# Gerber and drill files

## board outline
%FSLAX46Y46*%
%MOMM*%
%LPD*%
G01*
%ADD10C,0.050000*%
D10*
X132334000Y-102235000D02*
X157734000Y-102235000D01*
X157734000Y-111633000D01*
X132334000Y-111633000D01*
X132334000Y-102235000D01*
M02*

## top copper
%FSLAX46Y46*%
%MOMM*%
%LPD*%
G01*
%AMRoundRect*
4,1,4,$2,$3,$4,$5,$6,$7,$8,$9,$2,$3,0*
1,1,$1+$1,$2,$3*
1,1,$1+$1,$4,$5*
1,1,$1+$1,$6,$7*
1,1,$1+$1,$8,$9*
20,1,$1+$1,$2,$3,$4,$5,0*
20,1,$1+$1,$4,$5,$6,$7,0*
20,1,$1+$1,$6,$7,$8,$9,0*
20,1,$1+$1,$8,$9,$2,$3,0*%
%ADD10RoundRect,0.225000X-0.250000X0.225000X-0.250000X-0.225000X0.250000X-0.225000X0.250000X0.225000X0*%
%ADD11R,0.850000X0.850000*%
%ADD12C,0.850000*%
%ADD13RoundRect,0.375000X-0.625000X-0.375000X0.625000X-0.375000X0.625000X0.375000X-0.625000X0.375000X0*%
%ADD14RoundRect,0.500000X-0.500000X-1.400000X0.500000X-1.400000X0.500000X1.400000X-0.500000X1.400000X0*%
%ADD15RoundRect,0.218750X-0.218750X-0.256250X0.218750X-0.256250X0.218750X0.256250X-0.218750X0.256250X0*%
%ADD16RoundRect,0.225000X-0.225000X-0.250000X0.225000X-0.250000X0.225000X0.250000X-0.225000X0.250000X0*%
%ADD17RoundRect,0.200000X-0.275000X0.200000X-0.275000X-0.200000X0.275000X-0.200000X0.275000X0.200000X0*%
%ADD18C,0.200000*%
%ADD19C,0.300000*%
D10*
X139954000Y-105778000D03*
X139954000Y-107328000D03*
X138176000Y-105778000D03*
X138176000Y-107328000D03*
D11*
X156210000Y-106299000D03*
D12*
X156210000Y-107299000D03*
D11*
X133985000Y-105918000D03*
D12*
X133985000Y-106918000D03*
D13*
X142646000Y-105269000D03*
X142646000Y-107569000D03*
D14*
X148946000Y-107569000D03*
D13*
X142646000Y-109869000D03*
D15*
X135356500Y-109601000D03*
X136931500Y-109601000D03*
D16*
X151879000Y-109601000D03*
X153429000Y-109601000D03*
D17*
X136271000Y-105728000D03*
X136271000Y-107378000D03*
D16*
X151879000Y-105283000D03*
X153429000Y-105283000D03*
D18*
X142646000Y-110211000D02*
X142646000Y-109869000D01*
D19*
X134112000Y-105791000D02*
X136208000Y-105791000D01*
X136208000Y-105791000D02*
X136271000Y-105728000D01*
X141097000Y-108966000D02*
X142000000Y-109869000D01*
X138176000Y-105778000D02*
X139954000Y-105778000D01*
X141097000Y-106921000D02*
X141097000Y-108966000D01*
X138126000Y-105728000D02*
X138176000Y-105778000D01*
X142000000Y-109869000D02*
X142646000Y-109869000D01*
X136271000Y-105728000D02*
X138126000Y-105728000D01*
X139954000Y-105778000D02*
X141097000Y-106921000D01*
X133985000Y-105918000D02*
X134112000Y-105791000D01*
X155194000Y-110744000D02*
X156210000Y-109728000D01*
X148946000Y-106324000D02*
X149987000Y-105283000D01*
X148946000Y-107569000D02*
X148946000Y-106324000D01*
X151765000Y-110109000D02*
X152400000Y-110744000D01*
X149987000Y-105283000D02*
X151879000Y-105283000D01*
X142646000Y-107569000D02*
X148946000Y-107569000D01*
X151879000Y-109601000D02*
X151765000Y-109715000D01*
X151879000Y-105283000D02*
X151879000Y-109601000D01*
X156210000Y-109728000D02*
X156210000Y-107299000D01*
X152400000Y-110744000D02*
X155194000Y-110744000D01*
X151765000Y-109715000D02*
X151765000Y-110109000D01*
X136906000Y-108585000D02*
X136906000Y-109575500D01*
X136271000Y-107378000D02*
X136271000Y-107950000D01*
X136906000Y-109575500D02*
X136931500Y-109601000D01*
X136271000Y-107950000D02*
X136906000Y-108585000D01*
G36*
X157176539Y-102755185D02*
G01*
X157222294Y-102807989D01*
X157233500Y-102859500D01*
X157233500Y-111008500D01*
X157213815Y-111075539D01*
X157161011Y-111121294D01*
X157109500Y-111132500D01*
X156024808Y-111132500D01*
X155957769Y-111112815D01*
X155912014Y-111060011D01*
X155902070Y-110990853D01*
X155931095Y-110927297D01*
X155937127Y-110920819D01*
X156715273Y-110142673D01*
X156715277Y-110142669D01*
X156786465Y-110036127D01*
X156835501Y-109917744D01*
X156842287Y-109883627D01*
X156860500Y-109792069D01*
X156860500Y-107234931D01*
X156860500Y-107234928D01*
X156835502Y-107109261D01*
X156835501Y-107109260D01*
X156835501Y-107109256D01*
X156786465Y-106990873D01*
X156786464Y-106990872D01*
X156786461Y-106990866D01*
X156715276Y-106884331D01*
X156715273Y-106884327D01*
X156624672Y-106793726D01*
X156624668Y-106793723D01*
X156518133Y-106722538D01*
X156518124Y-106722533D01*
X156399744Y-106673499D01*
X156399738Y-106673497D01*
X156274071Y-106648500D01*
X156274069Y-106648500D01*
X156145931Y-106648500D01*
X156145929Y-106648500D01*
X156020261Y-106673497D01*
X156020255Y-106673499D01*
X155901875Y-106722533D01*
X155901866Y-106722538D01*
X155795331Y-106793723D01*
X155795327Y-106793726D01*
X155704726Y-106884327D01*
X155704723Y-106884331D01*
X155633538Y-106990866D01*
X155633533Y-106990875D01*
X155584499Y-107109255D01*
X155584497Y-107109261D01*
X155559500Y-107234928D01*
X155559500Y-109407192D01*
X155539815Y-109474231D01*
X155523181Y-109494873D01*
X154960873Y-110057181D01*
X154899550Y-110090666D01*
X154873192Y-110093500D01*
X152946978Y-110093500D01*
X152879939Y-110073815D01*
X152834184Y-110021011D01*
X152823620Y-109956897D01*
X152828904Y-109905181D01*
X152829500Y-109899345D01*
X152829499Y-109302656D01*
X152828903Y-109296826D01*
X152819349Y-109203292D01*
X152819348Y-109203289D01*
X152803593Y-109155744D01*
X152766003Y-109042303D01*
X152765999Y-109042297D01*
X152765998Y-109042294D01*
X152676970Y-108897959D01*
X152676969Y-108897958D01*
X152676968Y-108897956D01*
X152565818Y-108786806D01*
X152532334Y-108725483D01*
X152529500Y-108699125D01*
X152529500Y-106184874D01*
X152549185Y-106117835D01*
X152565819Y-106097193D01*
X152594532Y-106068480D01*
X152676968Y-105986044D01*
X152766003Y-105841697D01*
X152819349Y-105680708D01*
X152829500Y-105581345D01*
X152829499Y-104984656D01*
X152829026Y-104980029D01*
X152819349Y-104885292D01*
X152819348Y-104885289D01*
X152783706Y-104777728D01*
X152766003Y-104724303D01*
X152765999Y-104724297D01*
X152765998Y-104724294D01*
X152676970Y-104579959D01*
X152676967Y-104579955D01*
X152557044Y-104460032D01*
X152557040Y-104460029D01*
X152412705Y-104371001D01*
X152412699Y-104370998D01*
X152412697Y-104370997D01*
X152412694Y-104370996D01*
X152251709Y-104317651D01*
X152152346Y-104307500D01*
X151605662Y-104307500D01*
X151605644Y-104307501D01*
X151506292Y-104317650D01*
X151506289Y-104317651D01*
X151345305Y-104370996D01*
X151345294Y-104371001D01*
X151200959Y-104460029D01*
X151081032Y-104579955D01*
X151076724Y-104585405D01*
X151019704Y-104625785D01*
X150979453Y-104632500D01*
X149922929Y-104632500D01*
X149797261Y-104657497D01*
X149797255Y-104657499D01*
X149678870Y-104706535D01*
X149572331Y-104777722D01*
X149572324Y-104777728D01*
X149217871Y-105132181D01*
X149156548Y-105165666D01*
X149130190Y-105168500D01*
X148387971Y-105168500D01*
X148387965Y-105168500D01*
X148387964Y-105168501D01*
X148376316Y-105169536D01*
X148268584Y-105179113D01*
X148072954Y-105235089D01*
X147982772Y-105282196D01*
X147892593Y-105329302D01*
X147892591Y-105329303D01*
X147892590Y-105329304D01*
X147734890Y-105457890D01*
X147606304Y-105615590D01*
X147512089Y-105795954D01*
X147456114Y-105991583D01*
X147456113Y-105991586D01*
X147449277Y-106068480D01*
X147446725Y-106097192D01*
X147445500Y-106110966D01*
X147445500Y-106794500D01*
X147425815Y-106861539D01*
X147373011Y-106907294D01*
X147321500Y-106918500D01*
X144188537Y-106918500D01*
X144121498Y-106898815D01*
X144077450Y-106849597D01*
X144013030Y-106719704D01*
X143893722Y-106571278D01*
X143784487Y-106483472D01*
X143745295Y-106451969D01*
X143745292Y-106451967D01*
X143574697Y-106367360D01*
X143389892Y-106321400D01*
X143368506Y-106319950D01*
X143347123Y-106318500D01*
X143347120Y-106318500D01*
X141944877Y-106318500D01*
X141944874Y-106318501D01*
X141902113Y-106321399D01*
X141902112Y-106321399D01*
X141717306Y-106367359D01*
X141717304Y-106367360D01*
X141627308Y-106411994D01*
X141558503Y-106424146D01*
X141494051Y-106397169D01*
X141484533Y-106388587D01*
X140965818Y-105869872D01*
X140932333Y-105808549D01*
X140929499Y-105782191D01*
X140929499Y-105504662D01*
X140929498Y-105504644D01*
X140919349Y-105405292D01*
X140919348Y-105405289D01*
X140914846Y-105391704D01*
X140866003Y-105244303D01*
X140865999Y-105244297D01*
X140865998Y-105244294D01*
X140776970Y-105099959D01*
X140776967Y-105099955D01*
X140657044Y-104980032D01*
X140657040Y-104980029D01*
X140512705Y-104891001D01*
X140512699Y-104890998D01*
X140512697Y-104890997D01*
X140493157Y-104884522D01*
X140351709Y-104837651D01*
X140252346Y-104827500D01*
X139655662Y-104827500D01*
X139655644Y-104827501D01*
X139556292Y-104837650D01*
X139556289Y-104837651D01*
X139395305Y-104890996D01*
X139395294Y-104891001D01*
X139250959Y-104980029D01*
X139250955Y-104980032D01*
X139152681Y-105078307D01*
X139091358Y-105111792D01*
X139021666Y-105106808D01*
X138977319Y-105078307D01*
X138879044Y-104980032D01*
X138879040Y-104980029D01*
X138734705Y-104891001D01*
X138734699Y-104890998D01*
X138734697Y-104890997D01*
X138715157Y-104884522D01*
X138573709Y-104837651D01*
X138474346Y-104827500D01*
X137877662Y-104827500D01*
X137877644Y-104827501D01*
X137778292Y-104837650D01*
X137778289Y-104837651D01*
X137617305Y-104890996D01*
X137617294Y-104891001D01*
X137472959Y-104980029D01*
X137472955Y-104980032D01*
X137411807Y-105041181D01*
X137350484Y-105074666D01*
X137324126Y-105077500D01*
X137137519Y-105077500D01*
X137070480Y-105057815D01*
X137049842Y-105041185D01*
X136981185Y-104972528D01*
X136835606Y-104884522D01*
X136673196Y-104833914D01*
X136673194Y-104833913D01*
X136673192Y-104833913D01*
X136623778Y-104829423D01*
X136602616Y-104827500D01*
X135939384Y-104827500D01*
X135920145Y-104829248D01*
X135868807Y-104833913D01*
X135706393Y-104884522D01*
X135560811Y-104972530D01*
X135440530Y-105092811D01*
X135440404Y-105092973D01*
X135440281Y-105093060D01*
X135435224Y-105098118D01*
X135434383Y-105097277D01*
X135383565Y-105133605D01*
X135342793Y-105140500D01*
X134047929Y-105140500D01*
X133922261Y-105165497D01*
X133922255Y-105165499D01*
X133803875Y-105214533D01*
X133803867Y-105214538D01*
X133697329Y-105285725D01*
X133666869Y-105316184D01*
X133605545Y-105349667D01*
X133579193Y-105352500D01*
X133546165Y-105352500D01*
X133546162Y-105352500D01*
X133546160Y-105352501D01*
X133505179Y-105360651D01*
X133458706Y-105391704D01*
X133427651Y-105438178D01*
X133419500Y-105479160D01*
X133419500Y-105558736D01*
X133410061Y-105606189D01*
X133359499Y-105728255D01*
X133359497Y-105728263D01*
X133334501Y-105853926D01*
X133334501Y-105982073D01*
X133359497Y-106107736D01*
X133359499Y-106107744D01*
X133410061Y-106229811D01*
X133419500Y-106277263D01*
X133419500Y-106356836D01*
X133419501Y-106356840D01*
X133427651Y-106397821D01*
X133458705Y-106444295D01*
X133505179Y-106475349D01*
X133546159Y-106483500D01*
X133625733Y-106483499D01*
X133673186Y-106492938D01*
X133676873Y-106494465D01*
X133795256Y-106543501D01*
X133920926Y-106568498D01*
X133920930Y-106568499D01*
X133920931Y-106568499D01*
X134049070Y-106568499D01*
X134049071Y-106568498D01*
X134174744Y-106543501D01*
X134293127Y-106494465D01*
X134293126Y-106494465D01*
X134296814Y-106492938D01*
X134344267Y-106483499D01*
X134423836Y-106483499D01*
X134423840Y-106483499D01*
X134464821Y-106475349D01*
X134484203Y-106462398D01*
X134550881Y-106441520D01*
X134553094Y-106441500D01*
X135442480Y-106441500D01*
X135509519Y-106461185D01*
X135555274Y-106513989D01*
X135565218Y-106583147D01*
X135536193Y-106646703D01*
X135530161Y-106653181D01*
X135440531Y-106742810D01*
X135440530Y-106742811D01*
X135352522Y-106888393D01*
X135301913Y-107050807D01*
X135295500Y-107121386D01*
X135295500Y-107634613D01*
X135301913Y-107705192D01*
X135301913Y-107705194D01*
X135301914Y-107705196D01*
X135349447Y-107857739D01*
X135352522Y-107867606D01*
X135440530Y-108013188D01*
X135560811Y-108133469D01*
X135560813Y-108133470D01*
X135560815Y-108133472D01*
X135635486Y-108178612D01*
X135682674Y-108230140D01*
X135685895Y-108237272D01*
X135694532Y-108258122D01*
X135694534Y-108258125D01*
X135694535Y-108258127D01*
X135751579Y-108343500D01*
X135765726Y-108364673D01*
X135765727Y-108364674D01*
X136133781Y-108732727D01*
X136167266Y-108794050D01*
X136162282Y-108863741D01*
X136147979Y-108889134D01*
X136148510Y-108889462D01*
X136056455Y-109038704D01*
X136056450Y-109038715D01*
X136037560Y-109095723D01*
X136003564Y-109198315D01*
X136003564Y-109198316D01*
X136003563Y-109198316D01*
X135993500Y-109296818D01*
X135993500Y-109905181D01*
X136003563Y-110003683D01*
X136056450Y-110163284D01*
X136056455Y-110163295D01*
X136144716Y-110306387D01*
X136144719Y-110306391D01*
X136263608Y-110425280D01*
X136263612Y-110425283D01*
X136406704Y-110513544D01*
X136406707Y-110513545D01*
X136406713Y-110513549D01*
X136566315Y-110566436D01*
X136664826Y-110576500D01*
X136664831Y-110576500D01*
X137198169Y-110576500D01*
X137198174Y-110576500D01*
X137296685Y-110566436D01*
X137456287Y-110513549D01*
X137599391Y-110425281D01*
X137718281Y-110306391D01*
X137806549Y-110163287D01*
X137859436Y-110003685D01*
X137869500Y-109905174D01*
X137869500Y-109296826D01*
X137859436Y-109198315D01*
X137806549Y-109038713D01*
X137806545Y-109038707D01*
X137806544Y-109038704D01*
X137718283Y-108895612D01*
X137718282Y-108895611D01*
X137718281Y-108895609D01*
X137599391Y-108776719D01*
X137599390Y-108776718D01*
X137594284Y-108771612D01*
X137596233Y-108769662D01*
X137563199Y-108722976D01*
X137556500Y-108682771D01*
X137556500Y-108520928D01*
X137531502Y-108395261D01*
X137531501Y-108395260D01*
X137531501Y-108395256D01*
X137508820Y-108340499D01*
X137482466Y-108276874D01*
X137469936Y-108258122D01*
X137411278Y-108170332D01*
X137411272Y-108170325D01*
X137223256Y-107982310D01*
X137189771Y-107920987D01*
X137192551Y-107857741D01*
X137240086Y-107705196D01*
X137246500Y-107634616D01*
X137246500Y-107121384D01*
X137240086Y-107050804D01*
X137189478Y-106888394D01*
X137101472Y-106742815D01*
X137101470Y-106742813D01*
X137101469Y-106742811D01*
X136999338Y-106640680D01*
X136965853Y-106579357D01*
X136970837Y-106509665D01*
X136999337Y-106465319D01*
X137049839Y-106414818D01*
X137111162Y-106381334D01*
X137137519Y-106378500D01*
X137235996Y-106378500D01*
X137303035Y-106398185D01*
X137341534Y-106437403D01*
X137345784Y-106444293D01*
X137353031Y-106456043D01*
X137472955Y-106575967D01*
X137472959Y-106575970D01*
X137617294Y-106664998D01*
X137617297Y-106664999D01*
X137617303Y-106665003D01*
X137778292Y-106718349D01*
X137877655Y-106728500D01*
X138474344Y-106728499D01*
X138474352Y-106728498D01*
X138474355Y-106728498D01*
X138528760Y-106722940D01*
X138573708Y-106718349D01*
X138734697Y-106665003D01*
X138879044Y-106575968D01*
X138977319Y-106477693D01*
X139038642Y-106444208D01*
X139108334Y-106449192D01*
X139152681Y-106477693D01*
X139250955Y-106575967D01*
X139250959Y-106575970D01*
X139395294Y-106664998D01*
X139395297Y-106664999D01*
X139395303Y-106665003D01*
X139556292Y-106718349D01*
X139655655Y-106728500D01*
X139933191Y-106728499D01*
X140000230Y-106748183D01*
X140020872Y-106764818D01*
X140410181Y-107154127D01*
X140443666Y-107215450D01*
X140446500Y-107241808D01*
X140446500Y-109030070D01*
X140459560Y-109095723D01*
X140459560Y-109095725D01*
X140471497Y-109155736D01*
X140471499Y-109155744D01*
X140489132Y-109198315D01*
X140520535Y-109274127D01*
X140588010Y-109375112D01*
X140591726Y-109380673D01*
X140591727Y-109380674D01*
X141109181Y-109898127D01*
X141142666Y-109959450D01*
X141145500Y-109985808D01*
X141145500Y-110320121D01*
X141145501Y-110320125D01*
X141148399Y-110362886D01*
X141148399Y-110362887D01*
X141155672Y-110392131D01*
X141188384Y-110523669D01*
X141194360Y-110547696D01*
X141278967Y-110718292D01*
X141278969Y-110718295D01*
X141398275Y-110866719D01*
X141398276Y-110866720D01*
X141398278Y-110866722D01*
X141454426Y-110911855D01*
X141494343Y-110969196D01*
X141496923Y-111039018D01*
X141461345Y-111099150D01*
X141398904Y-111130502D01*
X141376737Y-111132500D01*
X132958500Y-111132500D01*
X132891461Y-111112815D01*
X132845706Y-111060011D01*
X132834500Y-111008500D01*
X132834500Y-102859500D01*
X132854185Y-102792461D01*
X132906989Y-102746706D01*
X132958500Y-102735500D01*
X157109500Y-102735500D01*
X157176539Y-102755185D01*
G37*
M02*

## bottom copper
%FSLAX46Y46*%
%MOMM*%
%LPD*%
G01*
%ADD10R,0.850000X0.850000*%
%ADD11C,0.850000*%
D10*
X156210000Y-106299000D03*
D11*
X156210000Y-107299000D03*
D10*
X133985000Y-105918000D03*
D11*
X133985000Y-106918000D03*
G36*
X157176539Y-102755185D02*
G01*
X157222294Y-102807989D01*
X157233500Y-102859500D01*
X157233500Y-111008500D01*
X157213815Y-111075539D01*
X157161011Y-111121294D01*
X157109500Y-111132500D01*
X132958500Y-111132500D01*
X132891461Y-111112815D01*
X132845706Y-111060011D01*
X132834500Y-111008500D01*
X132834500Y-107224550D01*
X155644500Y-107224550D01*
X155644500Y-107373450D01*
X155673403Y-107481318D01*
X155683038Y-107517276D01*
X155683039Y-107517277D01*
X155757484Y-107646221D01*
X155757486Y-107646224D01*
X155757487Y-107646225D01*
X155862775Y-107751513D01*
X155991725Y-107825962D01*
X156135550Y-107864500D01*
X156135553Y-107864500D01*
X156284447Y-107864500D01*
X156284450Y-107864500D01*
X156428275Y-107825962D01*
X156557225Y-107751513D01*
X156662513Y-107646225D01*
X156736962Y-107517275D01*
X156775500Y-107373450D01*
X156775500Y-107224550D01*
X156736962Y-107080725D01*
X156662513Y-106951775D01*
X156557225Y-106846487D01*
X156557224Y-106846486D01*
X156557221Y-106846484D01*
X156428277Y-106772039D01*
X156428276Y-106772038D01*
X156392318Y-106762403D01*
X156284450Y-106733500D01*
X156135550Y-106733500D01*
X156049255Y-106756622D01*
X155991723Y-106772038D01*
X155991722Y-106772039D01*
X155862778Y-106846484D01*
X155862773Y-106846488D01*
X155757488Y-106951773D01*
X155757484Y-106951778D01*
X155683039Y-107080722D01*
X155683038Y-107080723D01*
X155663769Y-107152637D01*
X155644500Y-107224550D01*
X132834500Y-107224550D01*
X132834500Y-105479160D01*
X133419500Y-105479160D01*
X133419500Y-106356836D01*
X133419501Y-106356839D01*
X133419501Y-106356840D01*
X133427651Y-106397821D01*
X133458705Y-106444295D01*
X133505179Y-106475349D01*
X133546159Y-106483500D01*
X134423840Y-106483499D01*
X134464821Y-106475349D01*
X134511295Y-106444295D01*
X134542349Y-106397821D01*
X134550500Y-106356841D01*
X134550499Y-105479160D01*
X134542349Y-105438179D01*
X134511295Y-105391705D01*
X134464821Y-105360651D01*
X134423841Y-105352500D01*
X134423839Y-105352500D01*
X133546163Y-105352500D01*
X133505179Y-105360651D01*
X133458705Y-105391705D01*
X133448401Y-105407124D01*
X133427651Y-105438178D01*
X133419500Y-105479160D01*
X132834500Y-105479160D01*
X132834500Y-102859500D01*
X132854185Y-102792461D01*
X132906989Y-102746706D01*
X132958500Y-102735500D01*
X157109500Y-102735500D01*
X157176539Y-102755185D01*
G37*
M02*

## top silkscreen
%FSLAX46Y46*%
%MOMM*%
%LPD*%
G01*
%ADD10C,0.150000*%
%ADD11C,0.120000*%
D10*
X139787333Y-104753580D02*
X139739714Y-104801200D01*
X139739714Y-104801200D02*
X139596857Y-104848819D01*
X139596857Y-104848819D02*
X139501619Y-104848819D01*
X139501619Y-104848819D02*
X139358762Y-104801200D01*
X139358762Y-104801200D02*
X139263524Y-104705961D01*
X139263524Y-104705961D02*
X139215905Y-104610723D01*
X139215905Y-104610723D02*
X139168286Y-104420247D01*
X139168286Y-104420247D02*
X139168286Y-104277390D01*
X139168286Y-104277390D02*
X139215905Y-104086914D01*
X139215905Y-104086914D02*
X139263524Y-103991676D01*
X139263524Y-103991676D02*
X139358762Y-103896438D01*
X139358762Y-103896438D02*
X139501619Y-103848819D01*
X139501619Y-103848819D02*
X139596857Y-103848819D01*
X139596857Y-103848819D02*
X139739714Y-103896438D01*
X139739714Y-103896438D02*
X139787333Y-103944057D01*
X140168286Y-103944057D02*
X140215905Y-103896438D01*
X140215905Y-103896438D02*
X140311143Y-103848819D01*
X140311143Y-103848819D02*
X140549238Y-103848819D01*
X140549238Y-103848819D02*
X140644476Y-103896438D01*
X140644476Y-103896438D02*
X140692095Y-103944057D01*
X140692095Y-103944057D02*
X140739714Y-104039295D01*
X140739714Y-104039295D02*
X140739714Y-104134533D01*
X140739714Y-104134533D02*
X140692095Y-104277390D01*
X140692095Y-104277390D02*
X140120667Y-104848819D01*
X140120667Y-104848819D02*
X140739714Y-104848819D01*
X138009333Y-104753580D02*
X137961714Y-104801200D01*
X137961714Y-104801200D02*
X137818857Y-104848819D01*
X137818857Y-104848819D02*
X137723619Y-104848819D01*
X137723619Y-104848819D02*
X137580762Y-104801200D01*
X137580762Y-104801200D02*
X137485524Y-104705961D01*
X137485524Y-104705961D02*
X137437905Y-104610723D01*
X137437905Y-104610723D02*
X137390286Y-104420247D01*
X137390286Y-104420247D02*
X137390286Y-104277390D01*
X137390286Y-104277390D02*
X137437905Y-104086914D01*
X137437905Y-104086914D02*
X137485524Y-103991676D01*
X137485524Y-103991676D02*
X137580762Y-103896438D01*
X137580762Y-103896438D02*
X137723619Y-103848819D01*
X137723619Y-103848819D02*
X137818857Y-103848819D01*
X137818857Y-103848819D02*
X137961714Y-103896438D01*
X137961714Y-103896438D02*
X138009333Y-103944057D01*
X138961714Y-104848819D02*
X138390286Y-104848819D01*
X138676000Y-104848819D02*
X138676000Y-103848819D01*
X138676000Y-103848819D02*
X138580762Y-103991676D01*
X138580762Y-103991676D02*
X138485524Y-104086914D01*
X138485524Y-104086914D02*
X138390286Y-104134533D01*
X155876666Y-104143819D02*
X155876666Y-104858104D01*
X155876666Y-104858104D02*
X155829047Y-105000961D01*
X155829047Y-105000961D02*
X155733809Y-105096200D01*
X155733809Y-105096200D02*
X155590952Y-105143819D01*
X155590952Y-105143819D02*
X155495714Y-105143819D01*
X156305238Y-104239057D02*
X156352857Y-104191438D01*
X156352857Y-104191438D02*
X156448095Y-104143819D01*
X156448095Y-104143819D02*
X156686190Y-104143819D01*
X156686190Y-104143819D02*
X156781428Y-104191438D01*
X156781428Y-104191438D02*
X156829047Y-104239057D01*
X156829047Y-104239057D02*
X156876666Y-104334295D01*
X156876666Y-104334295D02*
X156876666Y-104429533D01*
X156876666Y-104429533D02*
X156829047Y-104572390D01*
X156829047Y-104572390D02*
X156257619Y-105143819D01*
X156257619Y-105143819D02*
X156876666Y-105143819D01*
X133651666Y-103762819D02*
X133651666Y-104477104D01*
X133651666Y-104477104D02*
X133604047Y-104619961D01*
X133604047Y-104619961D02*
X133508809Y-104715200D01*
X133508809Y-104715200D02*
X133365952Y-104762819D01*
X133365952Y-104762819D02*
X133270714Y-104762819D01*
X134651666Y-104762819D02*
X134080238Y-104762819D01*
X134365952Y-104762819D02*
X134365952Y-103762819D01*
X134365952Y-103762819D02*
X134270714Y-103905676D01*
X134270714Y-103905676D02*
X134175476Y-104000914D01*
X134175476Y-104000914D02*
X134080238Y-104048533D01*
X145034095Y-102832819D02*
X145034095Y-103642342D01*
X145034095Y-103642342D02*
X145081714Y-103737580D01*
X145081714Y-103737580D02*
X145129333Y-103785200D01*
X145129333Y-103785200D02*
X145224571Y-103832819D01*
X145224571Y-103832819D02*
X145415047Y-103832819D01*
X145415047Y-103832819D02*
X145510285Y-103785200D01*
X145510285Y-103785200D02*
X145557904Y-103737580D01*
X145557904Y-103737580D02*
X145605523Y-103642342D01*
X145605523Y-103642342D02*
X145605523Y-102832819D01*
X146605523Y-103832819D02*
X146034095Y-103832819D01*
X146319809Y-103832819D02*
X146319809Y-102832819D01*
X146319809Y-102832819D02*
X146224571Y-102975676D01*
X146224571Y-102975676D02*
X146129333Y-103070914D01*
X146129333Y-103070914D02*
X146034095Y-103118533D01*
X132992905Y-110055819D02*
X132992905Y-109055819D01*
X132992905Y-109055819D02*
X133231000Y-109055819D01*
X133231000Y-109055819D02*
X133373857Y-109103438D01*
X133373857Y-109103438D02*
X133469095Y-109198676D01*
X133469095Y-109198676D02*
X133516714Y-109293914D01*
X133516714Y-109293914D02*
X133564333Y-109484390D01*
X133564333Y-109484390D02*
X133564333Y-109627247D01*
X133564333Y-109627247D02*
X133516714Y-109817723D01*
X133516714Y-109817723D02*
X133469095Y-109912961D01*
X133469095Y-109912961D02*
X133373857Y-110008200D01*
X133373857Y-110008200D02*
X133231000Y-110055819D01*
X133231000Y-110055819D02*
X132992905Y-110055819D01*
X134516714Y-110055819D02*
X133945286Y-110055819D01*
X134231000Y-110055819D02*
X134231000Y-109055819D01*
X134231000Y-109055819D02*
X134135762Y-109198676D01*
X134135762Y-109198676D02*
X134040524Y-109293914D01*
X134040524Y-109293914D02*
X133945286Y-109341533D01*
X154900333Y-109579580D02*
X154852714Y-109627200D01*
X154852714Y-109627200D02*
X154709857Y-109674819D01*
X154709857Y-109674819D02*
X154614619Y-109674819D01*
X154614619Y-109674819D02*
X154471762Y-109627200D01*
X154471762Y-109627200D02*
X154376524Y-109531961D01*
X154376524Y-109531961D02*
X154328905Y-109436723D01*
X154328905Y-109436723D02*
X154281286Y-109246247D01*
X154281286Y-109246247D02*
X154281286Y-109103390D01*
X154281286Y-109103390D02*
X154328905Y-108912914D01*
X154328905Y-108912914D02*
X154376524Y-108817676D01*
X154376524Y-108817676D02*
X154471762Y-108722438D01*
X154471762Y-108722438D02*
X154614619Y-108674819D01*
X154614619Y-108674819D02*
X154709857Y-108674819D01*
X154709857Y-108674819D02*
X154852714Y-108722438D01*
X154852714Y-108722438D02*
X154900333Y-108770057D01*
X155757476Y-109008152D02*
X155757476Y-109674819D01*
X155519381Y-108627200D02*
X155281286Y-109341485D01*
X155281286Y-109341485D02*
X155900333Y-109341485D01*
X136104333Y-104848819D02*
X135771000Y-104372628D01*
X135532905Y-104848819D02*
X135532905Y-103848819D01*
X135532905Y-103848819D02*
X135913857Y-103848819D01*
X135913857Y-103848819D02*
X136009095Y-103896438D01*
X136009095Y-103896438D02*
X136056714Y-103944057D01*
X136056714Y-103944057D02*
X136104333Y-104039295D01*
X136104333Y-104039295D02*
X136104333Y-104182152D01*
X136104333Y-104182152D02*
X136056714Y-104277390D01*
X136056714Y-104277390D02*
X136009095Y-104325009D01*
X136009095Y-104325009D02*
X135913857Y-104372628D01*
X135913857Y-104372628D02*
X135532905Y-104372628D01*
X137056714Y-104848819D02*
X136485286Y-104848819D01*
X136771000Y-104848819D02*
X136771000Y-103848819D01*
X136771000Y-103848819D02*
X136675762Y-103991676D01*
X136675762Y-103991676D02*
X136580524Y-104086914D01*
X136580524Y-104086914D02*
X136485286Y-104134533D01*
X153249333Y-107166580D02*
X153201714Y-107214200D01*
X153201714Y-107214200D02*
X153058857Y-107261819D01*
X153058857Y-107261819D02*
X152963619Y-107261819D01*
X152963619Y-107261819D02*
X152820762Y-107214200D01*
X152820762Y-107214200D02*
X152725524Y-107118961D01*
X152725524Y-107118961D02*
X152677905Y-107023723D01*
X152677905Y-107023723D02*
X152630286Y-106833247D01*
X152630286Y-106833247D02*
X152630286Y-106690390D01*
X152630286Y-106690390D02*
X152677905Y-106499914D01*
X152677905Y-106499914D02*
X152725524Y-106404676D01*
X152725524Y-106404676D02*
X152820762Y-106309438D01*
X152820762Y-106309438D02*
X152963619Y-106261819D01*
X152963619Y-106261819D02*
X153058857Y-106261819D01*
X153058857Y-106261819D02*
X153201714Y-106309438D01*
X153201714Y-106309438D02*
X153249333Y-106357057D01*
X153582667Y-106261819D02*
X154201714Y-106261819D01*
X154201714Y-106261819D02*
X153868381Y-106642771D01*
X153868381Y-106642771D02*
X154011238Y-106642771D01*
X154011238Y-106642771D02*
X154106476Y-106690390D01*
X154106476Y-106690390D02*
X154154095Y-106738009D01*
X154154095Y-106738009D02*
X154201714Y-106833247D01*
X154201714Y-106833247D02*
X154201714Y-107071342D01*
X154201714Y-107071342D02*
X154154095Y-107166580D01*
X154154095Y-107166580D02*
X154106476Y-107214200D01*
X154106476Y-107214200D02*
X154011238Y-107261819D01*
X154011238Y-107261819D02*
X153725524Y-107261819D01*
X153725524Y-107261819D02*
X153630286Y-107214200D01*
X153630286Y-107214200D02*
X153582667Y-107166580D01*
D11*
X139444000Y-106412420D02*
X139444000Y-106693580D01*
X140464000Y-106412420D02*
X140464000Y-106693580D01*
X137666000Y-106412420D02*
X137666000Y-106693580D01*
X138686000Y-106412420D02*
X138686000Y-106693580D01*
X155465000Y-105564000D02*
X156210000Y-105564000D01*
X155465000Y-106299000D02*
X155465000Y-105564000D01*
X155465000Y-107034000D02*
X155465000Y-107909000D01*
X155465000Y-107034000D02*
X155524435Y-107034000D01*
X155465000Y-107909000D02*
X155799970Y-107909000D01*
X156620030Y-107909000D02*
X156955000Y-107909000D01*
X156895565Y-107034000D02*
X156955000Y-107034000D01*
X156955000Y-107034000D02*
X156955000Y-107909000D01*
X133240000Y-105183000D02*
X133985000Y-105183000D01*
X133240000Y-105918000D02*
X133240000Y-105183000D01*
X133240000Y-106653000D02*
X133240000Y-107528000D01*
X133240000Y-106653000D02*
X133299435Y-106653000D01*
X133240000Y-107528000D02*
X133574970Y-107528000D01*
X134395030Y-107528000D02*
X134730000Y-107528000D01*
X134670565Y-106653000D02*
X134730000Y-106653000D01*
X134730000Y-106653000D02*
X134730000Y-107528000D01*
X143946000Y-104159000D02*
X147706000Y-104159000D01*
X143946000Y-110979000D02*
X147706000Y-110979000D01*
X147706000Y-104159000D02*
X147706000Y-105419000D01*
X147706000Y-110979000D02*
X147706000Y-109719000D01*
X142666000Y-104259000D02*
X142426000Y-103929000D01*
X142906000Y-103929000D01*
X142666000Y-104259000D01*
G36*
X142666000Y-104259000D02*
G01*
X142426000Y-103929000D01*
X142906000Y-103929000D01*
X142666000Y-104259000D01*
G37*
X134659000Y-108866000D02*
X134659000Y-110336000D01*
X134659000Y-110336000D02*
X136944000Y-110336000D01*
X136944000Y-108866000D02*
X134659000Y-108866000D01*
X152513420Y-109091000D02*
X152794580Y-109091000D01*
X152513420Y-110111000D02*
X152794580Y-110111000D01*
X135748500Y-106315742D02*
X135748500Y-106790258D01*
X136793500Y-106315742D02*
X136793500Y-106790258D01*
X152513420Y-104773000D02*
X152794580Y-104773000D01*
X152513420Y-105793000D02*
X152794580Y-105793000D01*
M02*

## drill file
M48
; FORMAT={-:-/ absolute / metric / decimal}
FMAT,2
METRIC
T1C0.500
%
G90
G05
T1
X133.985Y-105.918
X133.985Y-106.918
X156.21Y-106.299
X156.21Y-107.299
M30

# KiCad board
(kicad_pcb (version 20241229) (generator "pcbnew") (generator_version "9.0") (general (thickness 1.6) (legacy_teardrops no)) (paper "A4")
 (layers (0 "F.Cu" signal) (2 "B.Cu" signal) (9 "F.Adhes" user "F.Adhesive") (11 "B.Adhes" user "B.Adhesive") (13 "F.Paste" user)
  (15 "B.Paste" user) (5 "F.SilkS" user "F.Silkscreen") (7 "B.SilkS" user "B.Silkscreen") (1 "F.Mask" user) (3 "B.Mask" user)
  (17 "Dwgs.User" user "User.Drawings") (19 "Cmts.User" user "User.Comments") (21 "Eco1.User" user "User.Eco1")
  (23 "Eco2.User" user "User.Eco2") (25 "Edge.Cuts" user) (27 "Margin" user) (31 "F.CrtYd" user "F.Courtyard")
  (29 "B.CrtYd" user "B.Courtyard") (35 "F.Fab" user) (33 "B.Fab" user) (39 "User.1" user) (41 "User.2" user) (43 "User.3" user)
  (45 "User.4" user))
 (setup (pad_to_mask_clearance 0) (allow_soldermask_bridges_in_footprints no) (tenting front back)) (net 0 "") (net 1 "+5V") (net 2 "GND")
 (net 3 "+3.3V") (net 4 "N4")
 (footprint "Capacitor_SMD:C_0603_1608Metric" (layer "F.Cu") (at 139.954 106.553 -90)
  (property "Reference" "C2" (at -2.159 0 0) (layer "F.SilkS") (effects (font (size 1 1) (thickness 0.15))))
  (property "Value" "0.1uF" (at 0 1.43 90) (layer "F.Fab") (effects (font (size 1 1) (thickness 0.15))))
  (fp_line (start -0.14058 0.51) (end 0.14058 0.51) (stroke (width 0.12) (type solid)) (layer "F.SilkS"))
  (fp_line (start -0.14058 -0.51) (end 0.14058 -0.51) (stroke (width 0.12) (type solid)) (layer "F.SilkS"))
  (pad "1" smd roundrect (at -0.775 0 270) (size 0.9 0.95) (layers "F.Cu" "F.Mask" "F.Paste") (roundrect_rratio 0.25) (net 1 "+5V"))
  (pad "2" smd roundrect (at 0.775 0 270) (size 0.9 0.95) (layers "F.Cu" "F.Mask" "F.Paste") (roundrect_rratio 0.25) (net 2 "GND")))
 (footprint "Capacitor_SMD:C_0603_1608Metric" (layer "F.Cu") (at 138.176 106.553 -90)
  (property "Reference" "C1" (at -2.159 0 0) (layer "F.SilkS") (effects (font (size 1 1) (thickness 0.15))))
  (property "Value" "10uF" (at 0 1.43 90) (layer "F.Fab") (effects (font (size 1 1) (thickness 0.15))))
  (fp_line (start -0.14058 0.51) (end 0.14058 0.51) (stroke (width 0.12) (type solid)) (layer "F.SilkS"))
  (fp_line (start -0.14058 -0.51) (end 0.14058 -0.51) (stroke (width 0.12) (type solid)) (layer "F.SilkS"))
  (pad "1" smd roundrect (at -0.775 0 270) (size 0.9 0.95) (layers "F.Cu" "F.Mask" "F.Paste") (roundrect_rratio 0.25) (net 1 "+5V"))
  (pad "2" smd roundrect (at 0.775 0 270) (size 0.9 0.95) (layers "F.Cu" "F.Mask" "F.Paste") (roundrect_rratio 0.25) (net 2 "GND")))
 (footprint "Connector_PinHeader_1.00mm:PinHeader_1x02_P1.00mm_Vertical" (layer "F.Cu") (at 156.21 106.299)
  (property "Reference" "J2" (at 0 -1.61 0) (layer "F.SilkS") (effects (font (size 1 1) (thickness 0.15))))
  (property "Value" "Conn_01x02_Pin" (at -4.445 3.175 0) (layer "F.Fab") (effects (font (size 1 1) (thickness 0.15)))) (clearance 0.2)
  (fp_line (start -0.745 -0.735) (end 0 -0.735) (stroke (width 0.12) (type solid)) (layer "F.SilkS"))
  (fp_line (start -0.745 0) (end -0.745 -0.735) (stroke (width 0.12) (type solid)) (layer "F.SilkS"))
  (fp_line (start -0.745 0.735) (end -0.745 1.61) (stroke (width 0.12) (type solid)) (layer "F.SilkS"))
  (fp_line (start -0.745 0.735) (end -0.685565 0.735) (stroke (width 0.12) (type solid)) (layer "F.SilkS"))
  (fp_line (start -0.745 1.61) (end -0.41003 1.61) (stroke (width 0.12) (type solid)) (layer "F.SilkS"))
  (fp_line (start 0.41003 1.61) (end 0.745 1.61) (stroke (width 0.12) (type solid)) (layer "F.SilkS"))
  (fp_line (start 0.685565 0.735) (end 0.745 0.735) (stroke (width 0.12) (type solid)) (layer "F.SilkS"))
  (fp_line (start 0.745 0.735) (end 0.745 1.61) (stroke (width 0.12) (type solid)) (layer "F.SilkS"))
  (pad "1" thru_hole rect (at 0 0) (size 0.85 0.85) (drill 0.5) (layers "*.Cu" "*.Mask") (remove_unused_layers no) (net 2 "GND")
   (clearance 0.14))
  (pad "2" thru_hole circle (at 0 1) (size 0.85 0.85) (drill 0.5) (layers "*.Cu" "*.Mask") (remove_unused_layers no) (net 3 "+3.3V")
   (clearance 0.14)))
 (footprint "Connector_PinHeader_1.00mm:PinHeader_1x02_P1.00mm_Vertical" (layer "F.Cu") (at 133.985 105.918)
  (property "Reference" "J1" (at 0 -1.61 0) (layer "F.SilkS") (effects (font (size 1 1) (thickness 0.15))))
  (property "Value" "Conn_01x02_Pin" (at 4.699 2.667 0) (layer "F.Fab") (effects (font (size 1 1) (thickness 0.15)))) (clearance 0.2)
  (fp_line (start -0.745 -0.735) (end 0 -0.735) (stroke (width 0.12) (type solid)) (layer "F.SilkS"))
  (fp_line (start -0.745 0) (end -0.745 -0.735) (stroke (width 0.12) (type solid)) (layer "F.SilkS"))
  (fp_line (start -0.745 0.735) (end -0.745 1.61) (stroke (width 0.12) (type solid)) (layer "F.SilkS"))
  (fp_line (start -0.745 0.735) (end -0.685565 0.735) (stroke (width 0.12) (type solid)) (layer "F.SilkS"))
  (fp_line (start -0.745 1.61) (end -0.41003 1.61) (stroke (width 0.12) (type solid)) (layer "F.SilkS"))
  (fp_line (start 0.41003 1.61) (end 0.745 1.61) (stroke (width 0.12) (type solid)) (layer "F.SilkS"))
  (fp_line (start 0.685565 0.735) (end 0.745 0.735) (stroke (width 0.12) (type solid)) (layer "F.SilkS"))
  (fp_line (start 0.745 0.735) (end 0.745 1.61) (stroke (width 0.12) (type solid)) (layer "F.SilkS"))
  (pad "1" thru_hole rect (at 0 0) (size 0.85 0.85) (drill 0.5) (layers "*.Cu" "*.Mask") (remove_unused_layers no) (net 1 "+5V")
   (clearance 0.14))
  (pad "2" thru_hole circle (at 0 1) (size 0.85 0.85) (drill 0.5) (layers "*.Cu" "*.Mask") (remove_unused_layers no) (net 2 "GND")
   (clearance 0.14)))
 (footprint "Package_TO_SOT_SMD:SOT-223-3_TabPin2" (layer "F.Cu") (at 145.796 107.569)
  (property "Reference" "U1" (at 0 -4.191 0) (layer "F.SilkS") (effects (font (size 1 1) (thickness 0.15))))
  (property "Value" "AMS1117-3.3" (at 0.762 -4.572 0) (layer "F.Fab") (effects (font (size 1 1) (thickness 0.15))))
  (fp_line (start -1.85 -3.41) (end 1.91 -3.41) (stroke (width 0.12) (type solid)) (layer "F.SilkS"))
  (fp_line (start -1.85 3.41) (end 1.91 3.41) (stroke (width 0.12) (type solid)) (layer "F.SilkS"))
  (fp_line (start 1.91 -3.41) (end 1.91 -2.15) (stroke (width 0.12) (type solid)) (layer "F.SilkS"))
  (fp_line (start 1.91 3.41) (end 1.91 2.15) (stroke (width 0.12) (type solid)) (layer "F.SilkS"))
  (fp_poly
   (pts (xy -3.13 -3.31) (xy -3.37 -3.64) (xy -2.89 -3.64) (xy -3.13 -3.31)) (stroke (width 0.12) (type solid)) (fill yes) (layer "F.SilkS"))
  (pad "1" smd roundrect (at -3.15 -2.3) (size 2 1.5) (layers "F.Cu" "F.Mask" "F.Paste") (roundrect_rratio 0.25) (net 2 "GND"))
  (pad "2" smd roundrect (at -3.15 0) (size 2 1.5) (layers "F.Cu" "F.Mask" "F.Paste") (roundrect_rratio 0.25) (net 3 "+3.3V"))
  (pad "2" smd roundrect (at 3.15 0) (size 2 3.8) (layers "F.Cu" "F.Mask" "F.Paste") (roundrect_rratio 0.25) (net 3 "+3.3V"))
  (pad "3" smd roundrect (at -3.15 2.3) (size 2 1.5) (layers "F.Cu" "F.Mask" "F.Paste") (roundrect_rratio 0.25) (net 1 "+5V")))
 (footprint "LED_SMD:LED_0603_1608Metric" (layer "F.Cu") (at 136.144 109.601)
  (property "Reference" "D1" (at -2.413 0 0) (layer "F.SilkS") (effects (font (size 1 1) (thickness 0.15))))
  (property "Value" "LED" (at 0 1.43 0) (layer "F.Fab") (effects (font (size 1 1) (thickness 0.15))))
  (fp_line (start -1.485 -0.735) (end -1.485 0.735) (stroke (width 0.12) (type solid)) (layer "F.SilkS"))
  (fp_line (start -1.485 0.735) (end 0.8 0.735) (stroke (width 0.12) (type solid)) (layer "F.SilkS"))
  (fp_line (start 0.8 -0.735) (end -1.485 -0.735) (stroke (width 0.12) (type solid)) (layer "F.SilkS"))
  (pad "1" smd roundrect (at -0.7875 0) (size 0.875 0.95) (layers "F.Cu" "F.Mask" "F.Paste") (roundrect_rratio 0.25) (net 2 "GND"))
  (pad "2" smd roundrect (at 0.7875 0) (size 0.875 0.95) (layers "F.Cu" "F.Mask" "F.Paste") (roundrect_rratio 0.25) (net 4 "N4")))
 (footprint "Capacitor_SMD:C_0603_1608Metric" (layer "F.Cu") (at 152.654 109.601)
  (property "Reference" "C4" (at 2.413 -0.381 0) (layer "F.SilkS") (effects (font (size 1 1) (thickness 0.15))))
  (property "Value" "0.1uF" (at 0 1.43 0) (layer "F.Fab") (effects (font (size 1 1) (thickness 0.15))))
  (fp_line (start -0.14058 -0.51) (end 0.14058 -0.51) (stroke (width 0.12) (type solid)) (layer "F.SilkS"))
  (fp_line (start -0.14058 0.51) (end 0.14058 0.51) (stroke (width 0.12) (type solid)) (layer "F.SilkS"))
  (pad "1" smd roundrect (at -0.775 0) (size 0.9 0.95) (layers "F.Cu" "F.Mask" "F.Paste") (roundrect_rratio 0.25) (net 3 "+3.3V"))
  (pad "2" smd roundrect (at 0.775 0) (size 0.9 0.95) (layers "F.Cu" "F.Mask" "F.Paste") (roundrect_rratio 0.25) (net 2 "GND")))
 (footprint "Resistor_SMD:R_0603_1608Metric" (layer "F.Cu") (at 136.271 106.553 -90)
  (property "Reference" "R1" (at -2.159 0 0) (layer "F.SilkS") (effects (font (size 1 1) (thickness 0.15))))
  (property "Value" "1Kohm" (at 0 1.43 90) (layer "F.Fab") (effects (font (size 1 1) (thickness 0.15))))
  (fp_line (start -0.237258 0.5225) (end 0.237258 0.5225) (stroke (width 0.12) (type solid)) (layer "F.SilkS"))
  (fp_line (start -0.237258 -0.5225) (end 0.237258 -0.5225) (stroke (width 0.12) (type solid)) (layer "F.SilkS"))
  (pad "1" smd roundrect (at -0.825 0 270) (size 0.8 0.95) (layers "F.Cu" "F.Mask" "F.Paste") (roundrect_rratio 0.25) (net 1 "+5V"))
  (pad "2" smd roundrect (at 0.825 0 270) (size 0.8 0.95) (layers "F.Cu" "F.Mask" "F.Paste") (roundrect_rratio 0.25) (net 4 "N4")))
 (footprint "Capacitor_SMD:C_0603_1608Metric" (layer "F.Cu") (at 152.654 105.283)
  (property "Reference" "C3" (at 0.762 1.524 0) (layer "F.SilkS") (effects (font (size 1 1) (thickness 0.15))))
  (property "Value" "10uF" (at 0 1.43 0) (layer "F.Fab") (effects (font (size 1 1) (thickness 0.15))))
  (fp_line (start -0.14058 -0.51) (end 0.14058 -0.51) (stroke (width 0.12) (type solid)) (layer "F.SilkS"))
  (fp_line (start -0.14058 0.51) (end 0.14058 0.51) (stroke (width 0.12) (type solid)) (layer "F.SilkS"))
  (pad "1" smd roundrect (at -0.775 0) (size 0.9 0.95) (layers "F.Cu" "F.Mask" "F.Paste") (roundrect_rratio 0.25) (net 3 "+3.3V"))
  (pad "2" smd roundrect (at 0.775 0) (size 0.9 0.95) (layers "F.Cu" "F.Mask" "F.Paste") (roundrect_rratio 0.25) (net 2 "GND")))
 (gr_rect (start 132.334 102.235) (end 157.734 111.633) (stroke (width 0.05) (type default)) (fill no) (layer "Edge.Cuts"))
 (segment (start 142.646 110.211) (end 142.646 109.869) (width 0.2) (layer "F.Cu") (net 1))
 (segment (start 134.112 105.791) (end 136.208 105.791) (width 0.3) (layer "F.Cu") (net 1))
 (segment (start 136.208 105.791) (end 136.271 105.728) (width 0.3) (layer "F.Cu") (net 1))
 (segment (start 141.097 108.966) (end 142 109.869) (width 0.3) (layer "F.Cu") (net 1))
 (segment (start 138.176 105.778) (end 139.954 105.778) (width 0.3) (layer "F.Cu") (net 1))
 (segment (start 141.097 106.921) (end 141.097 108.966) (width 0.3) (layer "F.Cu") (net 1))
 (segment (start 138.126 105.728) (end 138.176 105.778) (width 0.3) (layer "F.Cu") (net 1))
 (segment (start 142 109.869) (end 142.646 109.869) (width 0.3) (layer "F.Cu") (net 1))
 (segment (start 136.271 105.728) (end 138.126 105.728) (width 0.3) (layer "F.Cu") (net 1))
 (segment (start 139.954 105.778) (end 141.097 106.921) (width 0.3) (layer "F.Cu") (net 1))
 (segment (start 133.985 105.918) (end 134.112 105.791) (width 0.3) (layer "F.Cu") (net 1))
 (segment (start 155.194 110.744) (end 156.21 109.728) (width 0.3) (layer "F.Cu") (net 3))
 (segment (start 148.946 106.324) (end 149.987 105.283) (width 0.3) (layer "F.Cu") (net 3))
 (segment (start 148.946 107.569) (end 148.946 106.324) (width 0.3) (layer "F.Cu") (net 3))
 (segment (start 151.765 110.109) (end 152.4 110.744) (width 0.3) (layer "F.Cu") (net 3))
 (segment (start 149.987 105.283) (end 151.879 105.283) (width 0.3) (layer "F.Cu") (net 3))
 (segment (start 142.646 107.569) (end 148.946 107.569) (width 0.3) (layer "F.Cu") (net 3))
 (segment (start 151.879 109.601) (end 151.765 109.715) (width 0.3) (layer "F.Cu") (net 3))
 (segment (start 151.879 105.283) (end 151.879 109.601) (width 0.3) (layer "F.Cu") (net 3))
 (segment (start 156.21 109.728) (end 156.21 107.299) (width 0.3) (layer "F.Cu") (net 3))
 (segment (start 152.4 110.744) (end 155.194 110.744) (width 0.3) (layer "F.Cu") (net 3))
 (segment (start 151.765 109.715) (end 151.765 110.109) (width 0.3) (layer "F.Cu") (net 3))
 (segment (start 136.906 108.585) (end 136.906 109.5755) (width 0.3) (layer "F.Cu") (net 4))
 (segment (start 136.271 107.378) (end 136.271 107.95) (width 0.3) (layer "F.Cu") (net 4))
 (segment (start 136.906 109.5755) (end 136.9315 109.601) (width 0.3) (layer "F.Cu") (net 4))
 (segment (start 136.271 107.95) (end 136.906 108.585) (width 0.3) (layer "F.Cu") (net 4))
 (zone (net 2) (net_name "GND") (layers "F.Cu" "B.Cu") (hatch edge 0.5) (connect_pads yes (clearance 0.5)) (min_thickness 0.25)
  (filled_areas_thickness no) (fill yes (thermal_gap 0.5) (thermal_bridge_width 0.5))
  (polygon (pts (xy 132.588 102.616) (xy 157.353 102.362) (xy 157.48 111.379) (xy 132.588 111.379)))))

